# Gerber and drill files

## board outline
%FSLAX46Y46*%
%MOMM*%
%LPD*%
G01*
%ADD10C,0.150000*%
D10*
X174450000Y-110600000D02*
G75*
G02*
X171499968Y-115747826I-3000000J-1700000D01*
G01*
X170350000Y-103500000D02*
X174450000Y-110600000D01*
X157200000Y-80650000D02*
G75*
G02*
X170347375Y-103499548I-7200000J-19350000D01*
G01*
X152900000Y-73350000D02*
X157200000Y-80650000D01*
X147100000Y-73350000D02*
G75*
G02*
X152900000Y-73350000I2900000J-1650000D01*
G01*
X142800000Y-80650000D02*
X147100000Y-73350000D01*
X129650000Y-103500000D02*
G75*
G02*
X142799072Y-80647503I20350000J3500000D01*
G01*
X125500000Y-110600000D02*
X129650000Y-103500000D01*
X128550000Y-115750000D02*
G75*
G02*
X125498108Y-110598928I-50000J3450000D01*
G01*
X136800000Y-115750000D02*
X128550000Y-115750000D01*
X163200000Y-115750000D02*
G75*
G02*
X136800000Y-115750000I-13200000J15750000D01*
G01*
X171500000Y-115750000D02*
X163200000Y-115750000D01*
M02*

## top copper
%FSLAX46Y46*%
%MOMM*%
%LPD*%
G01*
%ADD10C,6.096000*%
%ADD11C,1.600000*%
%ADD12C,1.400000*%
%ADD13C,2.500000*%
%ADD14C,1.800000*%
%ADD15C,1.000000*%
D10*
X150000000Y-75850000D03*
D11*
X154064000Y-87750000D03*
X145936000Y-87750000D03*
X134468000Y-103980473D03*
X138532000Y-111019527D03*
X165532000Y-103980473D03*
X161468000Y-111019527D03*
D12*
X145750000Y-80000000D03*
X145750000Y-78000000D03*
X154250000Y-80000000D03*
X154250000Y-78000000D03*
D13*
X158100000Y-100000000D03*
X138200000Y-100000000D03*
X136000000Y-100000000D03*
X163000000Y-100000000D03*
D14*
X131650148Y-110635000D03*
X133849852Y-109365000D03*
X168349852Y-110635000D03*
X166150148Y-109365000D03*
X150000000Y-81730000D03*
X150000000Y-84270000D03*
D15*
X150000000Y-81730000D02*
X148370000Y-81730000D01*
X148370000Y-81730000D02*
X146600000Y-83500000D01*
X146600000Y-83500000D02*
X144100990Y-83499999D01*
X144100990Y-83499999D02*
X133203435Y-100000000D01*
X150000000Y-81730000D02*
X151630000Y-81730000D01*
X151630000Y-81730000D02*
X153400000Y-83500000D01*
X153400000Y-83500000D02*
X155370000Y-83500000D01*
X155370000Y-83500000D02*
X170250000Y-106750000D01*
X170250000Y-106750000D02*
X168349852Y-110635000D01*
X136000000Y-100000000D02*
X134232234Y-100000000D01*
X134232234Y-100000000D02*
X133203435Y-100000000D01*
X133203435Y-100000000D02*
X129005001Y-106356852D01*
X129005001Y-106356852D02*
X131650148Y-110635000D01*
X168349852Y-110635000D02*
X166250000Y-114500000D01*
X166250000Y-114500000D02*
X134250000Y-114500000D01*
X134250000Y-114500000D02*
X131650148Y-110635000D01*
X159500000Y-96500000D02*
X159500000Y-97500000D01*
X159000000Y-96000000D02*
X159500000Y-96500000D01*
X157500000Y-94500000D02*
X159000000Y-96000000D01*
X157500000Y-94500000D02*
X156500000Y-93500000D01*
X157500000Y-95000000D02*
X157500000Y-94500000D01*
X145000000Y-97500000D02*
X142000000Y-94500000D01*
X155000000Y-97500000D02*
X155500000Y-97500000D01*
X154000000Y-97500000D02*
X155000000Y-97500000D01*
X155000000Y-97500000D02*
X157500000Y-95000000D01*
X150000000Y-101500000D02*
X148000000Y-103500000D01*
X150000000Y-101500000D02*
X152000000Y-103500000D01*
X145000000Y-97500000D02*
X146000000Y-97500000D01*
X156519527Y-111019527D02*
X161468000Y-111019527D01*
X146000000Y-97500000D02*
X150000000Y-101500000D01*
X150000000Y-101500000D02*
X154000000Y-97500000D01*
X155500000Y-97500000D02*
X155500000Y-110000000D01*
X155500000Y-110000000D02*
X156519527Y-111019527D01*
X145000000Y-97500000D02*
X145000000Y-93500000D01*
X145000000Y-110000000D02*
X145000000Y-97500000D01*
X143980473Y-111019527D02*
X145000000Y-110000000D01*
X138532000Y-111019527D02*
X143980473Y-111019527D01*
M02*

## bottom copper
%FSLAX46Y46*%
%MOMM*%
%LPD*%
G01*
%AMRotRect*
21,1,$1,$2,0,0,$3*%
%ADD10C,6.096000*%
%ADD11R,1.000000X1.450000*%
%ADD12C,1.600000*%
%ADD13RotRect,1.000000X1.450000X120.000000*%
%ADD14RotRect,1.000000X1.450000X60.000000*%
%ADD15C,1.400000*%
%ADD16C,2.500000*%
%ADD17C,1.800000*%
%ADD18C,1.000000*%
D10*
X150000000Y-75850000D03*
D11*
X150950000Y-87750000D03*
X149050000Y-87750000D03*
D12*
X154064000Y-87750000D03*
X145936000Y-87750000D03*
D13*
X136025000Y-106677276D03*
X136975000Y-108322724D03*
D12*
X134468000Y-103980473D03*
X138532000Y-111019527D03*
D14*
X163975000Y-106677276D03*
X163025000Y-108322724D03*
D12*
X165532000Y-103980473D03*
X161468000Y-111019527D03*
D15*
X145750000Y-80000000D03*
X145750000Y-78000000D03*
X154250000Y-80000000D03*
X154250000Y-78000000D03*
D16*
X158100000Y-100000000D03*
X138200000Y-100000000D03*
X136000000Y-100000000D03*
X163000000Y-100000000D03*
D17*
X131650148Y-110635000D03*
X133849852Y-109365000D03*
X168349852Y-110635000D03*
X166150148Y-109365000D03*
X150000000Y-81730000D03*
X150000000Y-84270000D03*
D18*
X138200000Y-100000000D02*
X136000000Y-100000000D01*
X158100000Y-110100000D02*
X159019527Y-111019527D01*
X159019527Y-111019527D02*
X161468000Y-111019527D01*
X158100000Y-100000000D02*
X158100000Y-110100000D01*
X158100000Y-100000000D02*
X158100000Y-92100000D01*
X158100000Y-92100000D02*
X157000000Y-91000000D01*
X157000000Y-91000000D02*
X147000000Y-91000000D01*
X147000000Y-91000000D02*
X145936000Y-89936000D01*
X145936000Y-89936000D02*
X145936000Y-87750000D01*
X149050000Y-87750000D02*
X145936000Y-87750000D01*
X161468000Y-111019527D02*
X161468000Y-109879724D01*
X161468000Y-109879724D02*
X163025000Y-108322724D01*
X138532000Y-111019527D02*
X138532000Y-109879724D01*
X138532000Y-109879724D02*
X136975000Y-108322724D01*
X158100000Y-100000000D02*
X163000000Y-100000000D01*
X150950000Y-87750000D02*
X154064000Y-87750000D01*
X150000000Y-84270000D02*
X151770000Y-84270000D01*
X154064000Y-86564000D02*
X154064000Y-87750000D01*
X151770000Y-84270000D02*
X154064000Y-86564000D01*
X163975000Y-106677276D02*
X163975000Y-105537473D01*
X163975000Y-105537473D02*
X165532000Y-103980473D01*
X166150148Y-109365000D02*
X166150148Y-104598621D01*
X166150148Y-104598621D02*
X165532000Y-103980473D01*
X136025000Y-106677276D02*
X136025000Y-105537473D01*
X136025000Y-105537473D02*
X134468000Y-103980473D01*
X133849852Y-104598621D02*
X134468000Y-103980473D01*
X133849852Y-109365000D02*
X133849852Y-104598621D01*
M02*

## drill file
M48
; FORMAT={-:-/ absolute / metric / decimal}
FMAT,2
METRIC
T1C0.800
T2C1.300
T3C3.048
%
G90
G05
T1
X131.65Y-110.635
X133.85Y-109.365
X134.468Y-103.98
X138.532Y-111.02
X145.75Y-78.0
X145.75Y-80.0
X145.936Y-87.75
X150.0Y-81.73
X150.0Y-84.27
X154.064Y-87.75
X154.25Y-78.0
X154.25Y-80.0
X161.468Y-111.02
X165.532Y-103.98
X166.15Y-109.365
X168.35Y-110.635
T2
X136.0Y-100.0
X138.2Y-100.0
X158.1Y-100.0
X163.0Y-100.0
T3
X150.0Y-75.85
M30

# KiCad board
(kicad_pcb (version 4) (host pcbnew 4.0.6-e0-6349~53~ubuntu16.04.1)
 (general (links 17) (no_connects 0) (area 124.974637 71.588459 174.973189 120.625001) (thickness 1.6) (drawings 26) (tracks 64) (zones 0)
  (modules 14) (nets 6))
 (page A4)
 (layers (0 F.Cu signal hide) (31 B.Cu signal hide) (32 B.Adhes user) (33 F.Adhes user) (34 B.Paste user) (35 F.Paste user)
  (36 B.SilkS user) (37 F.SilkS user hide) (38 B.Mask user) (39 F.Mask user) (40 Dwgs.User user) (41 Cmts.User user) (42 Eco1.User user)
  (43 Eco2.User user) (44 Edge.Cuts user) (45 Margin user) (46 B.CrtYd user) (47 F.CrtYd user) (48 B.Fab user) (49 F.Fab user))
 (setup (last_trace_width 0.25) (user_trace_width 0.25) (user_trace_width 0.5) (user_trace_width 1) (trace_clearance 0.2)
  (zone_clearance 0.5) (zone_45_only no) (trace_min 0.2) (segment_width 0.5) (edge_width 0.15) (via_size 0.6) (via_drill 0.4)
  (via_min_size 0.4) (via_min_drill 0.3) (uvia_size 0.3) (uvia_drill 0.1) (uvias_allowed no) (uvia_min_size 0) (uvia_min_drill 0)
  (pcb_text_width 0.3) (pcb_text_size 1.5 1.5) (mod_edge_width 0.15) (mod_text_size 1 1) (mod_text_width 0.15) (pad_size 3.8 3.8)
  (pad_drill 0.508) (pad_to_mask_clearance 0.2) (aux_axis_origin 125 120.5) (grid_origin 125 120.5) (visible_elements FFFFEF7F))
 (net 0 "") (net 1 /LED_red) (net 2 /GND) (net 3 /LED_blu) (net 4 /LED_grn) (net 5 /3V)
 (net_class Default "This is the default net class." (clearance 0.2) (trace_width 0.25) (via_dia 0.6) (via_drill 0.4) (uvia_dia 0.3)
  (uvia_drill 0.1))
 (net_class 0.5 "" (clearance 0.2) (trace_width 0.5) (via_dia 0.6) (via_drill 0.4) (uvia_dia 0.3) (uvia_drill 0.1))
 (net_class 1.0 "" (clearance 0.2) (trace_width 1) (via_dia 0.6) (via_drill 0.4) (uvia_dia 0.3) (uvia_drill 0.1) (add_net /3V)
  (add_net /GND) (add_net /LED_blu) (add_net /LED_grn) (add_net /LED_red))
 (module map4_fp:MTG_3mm (layer F.Cu) (at 150 75.85)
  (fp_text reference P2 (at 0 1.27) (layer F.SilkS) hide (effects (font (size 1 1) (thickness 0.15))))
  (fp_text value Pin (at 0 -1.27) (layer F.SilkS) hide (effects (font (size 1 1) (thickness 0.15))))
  (pad 1 thru_hole circle (at 0 0) (size 6.096 6.096) (drill 3.048) (layers *.Cu *.Mask F.SilkS)))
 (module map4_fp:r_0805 (layer B.Cu) (at 150 87.75)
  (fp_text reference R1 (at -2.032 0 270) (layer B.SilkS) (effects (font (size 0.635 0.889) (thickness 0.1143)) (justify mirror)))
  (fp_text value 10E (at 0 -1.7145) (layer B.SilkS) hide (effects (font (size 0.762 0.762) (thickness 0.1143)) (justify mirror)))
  (pad 2 smd rect (at 0.95 0) (size 1 1.45) (layers B.Cu B.Paste B.Mask) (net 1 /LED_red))
  (pad 1 smd rect (at -0.95 0) (size 1 1.45) (layers B.Cu B.Paste B.Mask) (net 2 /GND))
  (pad 2 thru_hole circle (at 4.064 0) (size 1.6 1.6) (drill 0.8) (layers *.Cu *.Mask B.SilkS) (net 1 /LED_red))
  (pad 1 thru_hole circle (at -4.064 0) (size 1.6 1.6) (drill 0.8) (layers *.Cu *.Mask B.SilkS) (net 2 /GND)))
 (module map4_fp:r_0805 (layer B.Cu) (at 136.5 107.5 120)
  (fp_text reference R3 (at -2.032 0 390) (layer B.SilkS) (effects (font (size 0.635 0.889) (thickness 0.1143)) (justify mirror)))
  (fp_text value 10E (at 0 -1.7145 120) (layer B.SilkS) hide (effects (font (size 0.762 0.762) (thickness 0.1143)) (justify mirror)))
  (pad 2 smd rect (at 0.95 0 120) (size 1 1.45) (layers B.Cu B.Paste B.Mask) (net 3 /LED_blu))
  (pad 1 smd rect (at -0.95 0 120) (size 1 1.45) (layers B.Cu B.Paste B.Mask) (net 2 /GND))
  (pad 2 thru_hole circle (at 4.064 0 120) (size 1.6 1.6) (drill 0.8) (layers *.Cu *.Mask B.SilkS) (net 3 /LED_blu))
  (pad 1 thru_hole circle (at -4.064 0 120) (size 1.6 1.6) (drill 0.8) (layers *.Cu *.Mask B.SilkS) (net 2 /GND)))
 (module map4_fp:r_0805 (layer B.Cu) (at 163.5 107.5 60)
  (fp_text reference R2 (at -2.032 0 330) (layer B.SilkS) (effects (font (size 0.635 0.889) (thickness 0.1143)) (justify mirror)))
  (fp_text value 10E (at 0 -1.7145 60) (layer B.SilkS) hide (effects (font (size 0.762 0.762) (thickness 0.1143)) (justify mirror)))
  (pad 2 smd rect (at 0.95 0 60) (size 1 1.45) (layers B.Cu B.Paste B.Mask) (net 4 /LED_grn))
  (pad 1 smd rect (at -0.95 0 60) (size 1 1.45) (layers B.Cu B.Paste B.Mask) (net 2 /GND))
  (pad 2 thru_hole circle (at 4.064 0 60) (size 1.6 1.6) (drill 0.8) (layers *.Cu *.Mask B.SilkS) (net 4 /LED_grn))
  (pad 1 thru_hole circle (at -4.064 0 60) (size 1.6 1.6) (drill 0.8) (layers *.Cu *.Mask B.SilkS) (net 2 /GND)))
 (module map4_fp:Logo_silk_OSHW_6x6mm (layer B.Cu) (at 150 107.5 180)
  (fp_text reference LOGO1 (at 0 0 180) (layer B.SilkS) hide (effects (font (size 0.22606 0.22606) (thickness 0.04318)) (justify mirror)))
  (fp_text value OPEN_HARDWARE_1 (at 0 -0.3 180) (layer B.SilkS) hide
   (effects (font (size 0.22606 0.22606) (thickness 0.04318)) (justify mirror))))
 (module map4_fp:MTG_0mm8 (layer F.Cu) (at 145.75 80)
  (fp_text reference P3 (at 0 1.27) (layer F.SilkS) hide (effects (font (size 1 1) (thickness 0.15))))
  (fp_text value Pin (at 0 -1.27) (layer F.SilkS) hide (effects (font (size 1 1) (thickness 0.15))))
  (pad 1 thru_hole circle (at 0 0) (size 1.4 1.4) (drill 0.8) (layers *.Cu *.Mask F.SilkS)))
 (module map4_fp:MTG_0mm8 (layer F.Cu) (at 145.75 78)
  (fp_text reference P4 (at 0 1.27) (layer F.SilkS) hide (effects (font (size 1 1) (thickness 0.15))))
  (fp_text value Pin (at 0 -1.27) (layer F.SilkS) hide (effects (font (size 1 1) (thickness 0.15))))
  (pad 1 thru_hole circle (at 0 0) (size 1.4 1.4) (drill 0.8) (layers *.Cu *.Mask F.SilkS)))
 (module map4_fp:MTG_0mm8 (layer F.Cu) (at 154.25 80)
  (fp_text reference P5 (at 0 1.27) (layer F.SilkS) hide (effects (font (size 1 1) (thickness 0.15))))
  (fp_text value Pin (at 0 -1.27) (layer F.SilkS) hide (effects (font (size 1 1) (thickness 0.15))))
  (pad 1 thru_hole circle (at 0 0) (size 1.4 1.4) (drill 0.8) (layers *.Cu *.Mask F.SilkS)))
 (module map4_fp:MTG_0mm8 (layer F.Cu) (at 154.25 78)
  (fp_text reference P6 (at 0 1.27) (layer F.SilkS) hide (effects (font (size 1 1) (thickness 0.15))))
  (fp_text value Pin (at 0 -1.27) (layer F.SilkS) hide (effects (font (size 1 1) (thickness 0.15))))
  (pad 1 thru_hole circle (at 0 0) (size 1.4 1.4) (drill 0.8) (layers *.Cu *.Mask F.SilkS)))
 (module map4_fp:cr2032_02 (layer B.Cu) (at 150 100 90)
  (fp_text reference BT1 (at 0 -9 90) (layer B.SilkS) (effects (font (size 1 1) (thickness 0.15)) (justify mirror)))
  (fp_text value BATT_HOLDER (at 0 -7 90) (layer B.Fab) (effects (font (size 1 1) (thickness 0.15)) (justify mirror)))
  (pad 2 thru_hole circle (at 0 8.1 90) (size 2.5 2.5) (drill 1.3) (layers *.Cu *.Mask B.SilkS) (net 2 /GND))
  (pad 1 thru_hole circle (at 0 -11.8 90) (size 2.5 2.5) (drill 1.3) (layers *.Cu *.Mask B.SilkS) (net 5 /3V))
  (pad 1 thru_hole circle (at 0 -14 90) (size 2.5 2.5) (drill 1.3) (layers *.Cu *.Mask B.SilkS) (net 5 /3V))
  (pad 2 thru_hole circle (at 0 13 90) (size 2.5 2.5) (drill 1.3) (layers *.Cu *.Mask B.SilkS) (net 2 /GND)))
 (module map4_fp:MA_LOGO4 (layer F.Cu) (at 150 97.5)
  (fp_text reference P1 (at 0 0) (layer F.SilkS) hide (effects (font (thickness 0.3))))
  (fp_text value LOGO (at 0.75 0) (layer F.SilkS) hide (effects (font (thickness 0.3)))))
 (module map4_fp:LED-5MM (layer F.Cu) (at 132.75 110 30)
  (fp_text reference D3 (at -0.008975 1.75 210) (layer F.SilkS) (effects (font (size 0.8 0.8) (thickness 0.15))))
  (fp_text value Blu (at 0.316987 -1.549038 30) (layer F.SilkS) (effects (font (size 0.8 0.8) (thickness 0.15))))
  (pad 1 thru_hole circle (at -1.27 0 30) (size 1.8 1.8) (drill 0.8) (layers *.Cu *.Mask F.SilkS) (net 5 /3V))
  (pad 2 thru_hole circle (at 1.27 0 30) (size 1.8 1.8) (drill 0.8) (layers *.Cu *.Mask F.SilkS) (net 3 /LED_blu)))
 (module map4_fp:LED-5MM (layer F.Cu) (at 167.25 110 150)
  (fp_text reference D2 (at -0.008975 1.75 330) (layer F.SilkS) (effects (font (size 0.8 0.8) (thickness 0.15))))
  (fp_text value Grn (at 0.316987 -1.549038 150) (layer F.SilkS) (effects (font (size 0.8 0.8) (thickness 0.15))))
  (pad 1 thru_hole circle (at -1.27 0 150) (size 1.8 1.8) (drill 0.8) (layers *.Cu *.Mask F.SilkS) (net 5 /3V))
  (pad 2 thru_hole circle (at 1.27 0 150) (size 1.8 1.8) (drill 0.8) (layers *.Cu *.Mask F.SilkS) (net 4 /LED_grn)))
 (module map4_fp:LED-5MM (layer F.Cu) (at 150 83 270)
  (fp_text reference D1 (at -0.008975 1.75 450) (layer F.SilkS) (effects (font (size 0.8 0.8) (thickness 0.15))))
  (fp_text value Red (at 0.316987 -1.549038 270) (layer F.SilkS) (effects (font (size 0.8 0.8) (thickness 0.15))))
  (pad 1 thru_hole circle (at -1.27 0 270) (size 1.8 1.8) (drill 0.8) (layers *.Cu *.Mask F.SilkS) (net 5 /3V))
  (pad 2 thru_hole circle (at 1.27 0 270) (size 1.8 1.8) (drill 0.8) (layers *.Cu *.Mask F.SilkS) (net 1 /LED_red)))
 (gr_arc (start 171.45 112.3) (end 174.45 110.6) (angle 118.7084745) (layer Edge.Cuts) (width 0.15))
 (gr_line (start 170.35 103.5) (end 174.45 110.6) (layer Edge.Cuts) (width 0.15))
 (gr_arc (start 150 100) (end 157.2 80.65) (angle 79.34895054) (layer Edge.Cuts) (width 0.15))
 (gr_line (start 152.9 73.35) (end 157.2 80.65) (layer Edge.Cuts) (width 0.15))
 (gr_arc (start 150 75) (end 147.1 73.35) (angle 120.7232391) (layer Edge.Cuts) (width 0.15))
 (gr_line (start 142.8 80.65) (end 147.1 73.35) (layer Edge.Cuts) (width 0.15))
 (gr_arc (start 150 100) (end 129.65 103.5) (angle 79.34895344) (layer Edge.Cuts) (width 0.15))
 (gr_line (start 125.5 110.6) (end 129.65 103.5) (layer Edge.Cuts) (width 0.15))
 (gr_arc (start 128.5 112.3) (end 128.55 115.75) (angle 120.3690896) (layer Edge.Cuts) (width 0.15))
 (gr_line (start 136.8 115.75) (end 128.55 115.75) (layer Edge.Cuts) (width 0.15))
 (gr_arc (start 150 100) (end 163.2 115.75) (angle 79.93242788) (layer Edge.Cuts) (width 0.15))
 (gr_line (start 171.5 115.75) (end 163.2 115.75) (layer Edge.Cuts) (width 0.15))
 (segment (start 150 81.73) (end 148.37 81.73) (width 1) (layer F.Cu) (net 5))
 (segment (start 148.37 81.73) (end 146.6 83.5) (width 1) (layer F.Cu) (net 5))
 (segment (start 146.6 83.5) (end 144.10099 83.499999) (width 1) (layer F.Cu) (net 5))
 (segment (start 144.10099 83.499999) (end 133.203435 100) (width 1) (layer F.Cu) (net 5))
 (segment (start 150 81.73) (end 151.63 81.73) (width 1) (layer F.Cu) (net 5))
 (segment (start 151.63 81.73) (end 153.4 83.5) (width 1) (layer F.Cu) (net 5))
 (segment (start 153.4 83.5) (end 155.37 83.5) (width 1) (layer F.Cu) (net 5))
 (segment (start 155.37 83.5) (end 170.25 106.75) (width 1) (layer F.Cu) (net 5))
 (segment (start 170.25 106.75) (end 168.349852 110.635) (width 1) (layer F.Cu) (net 5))
 (segment (start 136 100) (end 134.232234 100) (width 1) (layer F.Cu) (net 5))
 (segment (start 134.232234 100) (end 133.203435 100) (width 1) (layer F.Cu) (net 5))
 (segment (start 133.203435 100) (end 129.005001 106.356852) (width 1) (layer F.Cu) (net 5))
 (segment (start 138.2 100) (end 136 100) (width 1) (layer B.Cu) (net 5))
 (segment (start 129.005001 106.356852) (end 131.650148 110.635) (width 1) (layer F.Cu) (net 5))
 (segment (start 168.349852 110.635) (end 166.25 114.5) (width 1) (layer F.Cu) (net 5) (status 10))
 (segment (start 166.25 114.5) (end 134.25 114.5) (width 1) (layer F.Cu) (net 5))
 (segment (start 134.25 114.5) (end 131.650148 110.635) (width 1) (layer F.Cu) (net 5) (status 20))
 (segment (start 159.5 96.5) (end 159.5 97.5) (width 1) (layer F.Cu) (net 2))
 (segment (start 159 96) (end 159.5 96.5) (width 1) (layer F.Cu) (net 2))
 (segment (start 157.5 94.5) (end 159 96) (width 1) (layer F.Cu) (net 2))
 (segment (start 157.5 94.5) (end 156.5 93.5) (width 1) (layer F.Cu) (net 2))
 (segment (start 157.5 95) (end 157.5 94.5) (width 1) (layer F.Cu) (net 2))
 (segment (start 145 97.5) (end 142 94.5) (width 1) (layer F.Cu) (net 2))
 (segment (start 155 97.5) (end 155.5 97.5) (width 1) (layer F.Cu) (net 2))
 (segment (start 154 97.5) (end 155 97.5) (width 1) (layer F.Cu) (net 2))
 (segment (start 155 97.5) (end 157.5 95) (width 1) (layer F.Cu) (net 2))
 (segment (start 150 101.5) (end 148 103.5) (width 1) (layer F.Cu) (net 2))
 (segment (start 150 101.5) (end 152 103.5) (width 1) (layer F.Cu) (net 2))
 (segment (start 145 97.5) (end 146 97.5) (width 1) (layer F.Cu) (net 2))
 (segment (start 156.519527 111.019527) (end 161.468 111.019527) (width 1) (layer F.Cu) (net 2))
 (segment (start 146 97.5) (end 150 101.5) (width 1) (layer F.Cu) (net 2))
 (segment (start 150 101.5) (end 154 97.5) (width 1) (layer F.Cu) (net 2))
 (segment (start 155.5 97.5) (end 155.5 110) (width 1) (layer F.Cu) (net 2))
 (segment (start 155.5 110) (end 156.519527 111.019527) (width 1) (layer F.Cu) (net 2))
 (segment (start 145 97.5) (end 145 93.5) (width 1) (layer F.Cu) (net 2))
 (segment (start 145 110) (end 145 97.5) (width 1) (layer F.Cu) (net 2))
 (segment (start 143.980473 111.019527) (end 145 110) (width 1) (layer F.Cu) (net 2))
 (segment (start 138.532 111.019527) (end 143.980473 111.019527) (width 1) (layer F.Cu) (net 2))
 (segment (start 158.1 110.1) (end 159.019527 111.019527) (width 1) (layer B.Cu) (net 2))
 (segment (start 159.019527 111.019527) (end 161.468 111.019527) (width 1) (layer B.Cu) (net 2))
 (segment (start 158.1 100) (end 158.1 110.1) (width 1) (layer B.Cu) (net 2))
 (segment (start 158.1 100) (end 158.1 92.1) (width 1) (layer B.Cu) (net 2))
 (segment (start 158.1 92.1) (end 157 91) (width 1) (layer B.Cu) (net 2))
 (segment (start 157 91) (end 147 91) (width 1) (layer B.Cu) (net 2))
 (segment (start 147 91) (end 145.936 89.936) (width 1) (layer B.Cu) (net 2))
 (segment (start 145.936 89.936) (end 145.936 87.75) (width 1) (layer B.Cu) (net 2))
 (segment (start 149.05 87.75) (end 145.936 87.75) (width 1) (layer B.Cu) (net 2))
 (segment (start 161.468 111.019527) (end 161.468 109.879724) (width 1) (layer B.Cu) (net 2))
 (segment (start 161.468 109.879724) (end 163.025 108.322724) (width 1) (layer B.Cu) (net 2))
 (segment (start 138.532 111.019527) (end 138.532 109.879724) (width 1) (layer B.Cu) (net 2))
 (segment (start 138.532 109.879724) (end 136.975 108.322724) (width 1) (layer B.Cu) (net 2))
 (segment (start 158.1 100) (end 163 100) (width 1) (layer B.Cu) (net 2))
 (segment (start 150.95 87.75) (end 154.064 87.75) (width 1) (layer B.Cu) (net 1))
 (segment (start 150 84.27) (end 151.77 84.27) (width 1) (layer B.Cu) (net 1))
 (segment (start 154.064 86.564) (end 154.064 87.75) (width 1) (layer B.Cu) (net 1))
 (segment (start 151.77 84.27) (end 154.064 86.564) (width 1) (layer B.Cu) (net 1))
 (segment (start 163.975 106.677276) (end 163.975 105.537473) (width 1) (layer B.Cu) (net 4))
 (segment (start 163.975 105.537473) (end 165.532 103.980473) (width 1) (layer B.Cu) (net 4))
 (segment (start 166.150148 109.365) (end 166.150148 104.598621) (width 1) (layer B.Cu) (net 4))
 (segment (start 166.150148 104.598621) (end 165.532 103.980473) (width 1) (layer B.Cu) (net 4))
 (segment (start 136.025 106.677276) (end 136.025 105.537473) (width 1) (layer B.Cu) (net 3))
 (segment (start 136.025 105.537473) (end 134.468 103.980473) (width 1) (layer B.Cu) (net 3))
 (segment (start 133.849852 104.598621) (end 134.468 103.980473) (width 1) (layer B.Cu) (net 3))
 (segment (start 133.849852 109.365) (end 133.849852 104.598621) (width 1) (layer B.Cu) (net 3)))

